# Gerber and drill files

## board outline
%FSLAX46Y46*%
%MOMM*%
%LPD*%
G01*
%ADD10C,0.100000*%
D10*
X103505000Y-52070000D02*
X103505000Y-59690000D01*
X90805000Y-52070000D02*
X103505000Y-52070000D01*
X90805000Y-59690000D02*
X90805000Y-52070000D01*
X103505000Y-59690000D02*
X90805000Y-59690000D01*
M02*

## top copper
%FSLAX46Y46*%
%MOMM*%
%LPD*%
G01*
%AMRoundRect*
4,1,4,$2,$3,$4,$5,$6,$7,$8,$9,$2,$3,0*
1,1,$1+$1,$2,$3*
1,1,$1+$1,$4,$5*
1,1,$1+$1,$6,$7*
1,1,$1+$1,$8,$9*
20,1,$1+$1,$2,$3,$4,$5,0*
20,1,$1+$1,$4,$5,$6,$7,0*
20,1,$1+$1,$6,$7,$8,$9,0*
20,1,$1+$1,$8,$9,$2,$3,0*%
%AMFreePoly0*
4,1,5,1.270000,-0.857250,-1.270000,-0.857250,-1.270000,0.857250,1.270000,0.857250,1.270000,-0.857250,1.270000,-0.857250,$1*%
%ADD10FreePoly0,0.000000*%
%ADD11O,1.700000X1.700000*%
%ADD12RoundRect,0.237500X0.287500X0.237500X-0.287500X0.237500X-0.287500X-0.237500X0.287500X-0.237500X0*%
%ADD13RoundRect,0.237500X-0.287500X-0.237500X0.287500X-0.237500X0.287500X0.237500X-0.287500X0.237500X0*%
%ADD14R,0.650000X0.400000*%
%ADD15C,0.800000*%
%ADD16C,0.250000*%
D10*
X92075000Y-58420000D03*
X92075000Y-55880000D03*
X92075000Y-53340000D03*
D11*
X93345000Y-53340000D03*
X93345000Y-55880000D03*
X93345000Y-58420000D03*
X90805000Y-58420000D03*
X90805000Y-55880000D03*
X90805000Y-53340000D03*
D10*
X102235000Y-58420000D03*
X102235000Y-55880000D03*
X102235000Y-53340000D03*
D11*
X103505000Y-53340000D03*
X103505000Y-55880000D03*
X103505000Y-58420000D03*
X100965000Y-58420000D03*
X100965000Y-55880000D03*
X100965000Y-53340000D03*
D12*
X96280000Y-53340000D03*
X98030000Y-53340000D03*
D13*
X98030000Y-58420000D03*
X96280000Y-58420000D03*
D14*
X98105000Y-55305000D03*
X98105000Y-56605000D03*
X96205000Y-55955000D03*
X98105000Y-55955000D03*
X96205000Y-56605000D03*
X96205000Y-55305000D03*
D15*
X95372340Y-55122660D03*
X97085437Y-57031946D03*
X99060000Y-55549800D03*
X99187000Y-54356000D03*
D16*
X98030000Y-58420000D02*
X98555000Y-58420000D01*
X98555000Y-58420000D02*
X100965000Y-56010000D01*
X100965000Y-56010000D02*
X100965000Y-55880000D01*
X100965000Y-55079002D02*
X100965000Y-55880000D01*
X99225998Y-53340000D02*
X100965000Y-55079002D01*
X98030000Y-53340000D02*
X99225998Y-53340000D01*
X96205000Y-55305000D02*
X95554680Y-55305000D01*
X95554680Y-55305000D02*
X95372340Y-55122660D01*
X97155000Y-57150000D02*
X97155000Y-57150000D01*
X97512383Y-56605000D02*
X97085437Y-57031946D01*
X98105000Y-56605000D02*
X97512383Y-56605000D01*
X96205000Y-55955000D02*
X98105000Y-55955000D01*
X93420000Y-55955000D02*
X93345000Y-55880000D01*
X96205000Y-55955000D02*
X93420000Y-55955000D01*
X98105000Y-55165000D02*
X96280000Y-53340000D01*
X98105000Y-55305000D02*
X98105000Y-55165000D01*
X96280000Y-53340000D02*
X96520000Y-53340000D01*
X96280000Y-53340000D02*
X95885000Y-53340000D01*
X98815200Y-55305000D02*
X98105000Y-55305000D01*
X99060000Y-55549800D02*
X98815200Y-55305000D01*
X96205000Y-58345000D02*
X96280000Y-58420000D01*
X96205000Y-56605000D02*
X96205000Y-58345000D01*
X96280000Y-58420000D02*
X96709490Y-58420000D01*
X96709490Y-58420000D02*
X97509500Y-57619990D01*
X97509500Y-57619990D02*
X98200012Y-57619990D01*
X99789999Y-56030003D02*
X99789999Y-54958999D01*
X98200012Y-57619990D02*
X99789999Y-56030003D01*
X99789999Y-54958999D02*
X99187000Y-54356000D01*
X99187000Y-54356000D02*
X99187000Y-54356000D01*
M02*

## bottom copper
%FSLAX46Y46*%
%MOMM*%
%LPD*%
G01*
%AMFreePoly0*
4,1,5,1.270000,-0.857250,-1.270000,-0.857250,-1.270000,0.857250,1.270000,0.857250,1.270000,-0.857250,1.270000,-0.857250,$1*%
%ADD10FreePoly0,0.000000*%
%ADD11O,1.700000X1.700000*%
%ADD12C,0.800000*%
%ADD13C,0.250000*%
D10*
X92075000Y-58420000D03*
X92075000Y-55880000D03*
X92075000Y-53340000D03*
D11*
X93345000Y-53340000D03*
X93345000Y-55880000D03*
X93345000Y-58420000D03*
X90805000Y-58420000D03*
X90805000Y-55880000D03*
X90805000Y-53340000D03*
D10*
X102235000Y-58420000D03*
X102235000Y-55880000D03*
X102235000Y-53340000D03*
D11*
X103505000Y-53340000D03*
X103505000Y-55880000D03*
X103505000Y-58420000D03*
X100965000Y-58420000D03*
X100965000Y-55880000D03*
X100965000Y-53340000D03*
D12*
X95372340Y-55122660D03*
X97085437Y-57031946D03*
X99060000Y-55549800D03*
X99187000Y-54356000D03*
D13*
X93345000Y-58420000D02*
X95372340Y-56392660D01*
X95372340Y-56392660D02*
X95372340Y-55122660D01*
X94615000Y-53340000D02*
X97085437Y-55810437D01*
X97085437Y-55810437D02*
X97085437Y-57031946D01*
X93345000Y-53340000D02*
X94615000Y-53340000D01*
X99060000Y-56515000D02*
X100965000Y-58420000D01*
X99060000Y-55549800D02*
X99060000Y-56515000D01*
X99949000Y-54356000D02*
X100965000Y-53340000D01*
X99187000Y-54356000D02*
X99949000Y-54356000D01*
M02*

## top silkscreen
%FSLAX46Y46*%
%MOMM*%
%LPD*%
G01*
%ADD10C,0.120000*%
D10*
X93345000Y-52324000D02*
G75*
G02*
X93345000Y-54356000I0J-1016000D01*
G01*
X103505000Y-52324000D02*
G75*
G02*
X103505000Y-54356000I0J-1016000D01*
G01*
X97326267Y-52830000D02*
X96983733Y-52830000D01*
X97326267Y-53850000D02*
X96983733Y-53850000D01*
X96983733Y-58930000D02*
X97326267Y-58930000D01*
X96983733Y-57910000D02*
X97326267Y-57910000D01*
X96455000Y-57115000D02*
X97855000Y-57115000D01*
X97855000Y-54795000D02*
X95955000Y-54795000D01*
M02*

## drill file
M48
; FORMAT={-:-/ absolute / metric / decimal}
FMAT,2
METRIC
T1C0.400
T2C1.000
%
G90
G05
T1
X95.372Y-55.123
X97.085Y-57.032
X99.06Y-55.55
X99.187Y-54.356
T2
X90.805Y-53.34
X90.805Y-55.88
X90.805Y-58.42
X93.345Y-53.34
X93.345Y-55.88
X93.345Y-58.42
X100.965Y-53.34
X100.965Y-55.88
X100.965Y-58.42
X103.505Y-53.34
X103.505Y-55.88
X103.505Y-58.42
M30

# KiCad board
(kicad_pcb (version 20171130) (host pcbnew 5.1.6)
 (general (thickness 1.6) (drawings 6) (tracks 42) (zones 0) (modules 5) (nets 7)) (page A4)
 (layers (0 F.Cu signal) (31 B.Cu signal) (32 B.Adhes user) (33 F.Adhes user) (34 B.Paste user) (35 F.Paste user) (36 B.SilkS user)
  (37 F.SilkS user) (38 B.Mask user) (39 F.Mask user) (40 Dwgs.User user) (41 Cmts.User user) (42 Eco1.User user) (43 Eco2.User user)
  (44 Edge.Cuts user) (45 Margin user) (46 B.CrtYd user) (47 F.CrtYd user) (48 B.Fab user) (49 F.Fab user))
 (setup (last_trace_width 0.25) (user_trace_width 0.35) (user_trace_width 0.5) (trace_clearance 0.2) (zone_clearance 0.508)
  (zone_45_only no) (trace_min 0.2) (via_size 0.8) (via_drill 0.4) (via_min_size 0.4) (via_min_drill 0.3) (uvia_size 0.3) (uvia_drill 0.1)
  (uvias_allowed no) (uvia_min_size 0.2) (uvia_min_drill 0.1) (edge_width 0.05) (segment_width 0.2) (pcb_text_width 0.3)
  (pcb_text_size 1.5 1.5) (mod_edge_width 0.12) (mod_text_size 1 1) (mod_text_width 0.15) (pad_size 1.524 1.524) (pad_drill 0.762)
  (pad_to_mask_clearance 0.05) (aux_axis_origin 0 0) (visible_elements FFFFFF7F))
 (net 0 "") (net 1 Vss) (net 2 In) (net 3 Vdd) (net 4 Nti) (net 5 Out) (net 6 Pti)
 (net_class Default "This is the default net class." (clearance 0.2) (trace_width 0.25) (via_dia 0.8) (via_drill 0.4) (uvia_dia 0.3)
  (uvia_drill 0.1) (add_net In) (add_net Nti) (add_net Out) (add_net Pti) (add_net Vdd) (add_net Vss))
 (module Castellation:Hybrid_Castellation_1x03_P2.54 (layer F.Cu) (at 92.075 53.34)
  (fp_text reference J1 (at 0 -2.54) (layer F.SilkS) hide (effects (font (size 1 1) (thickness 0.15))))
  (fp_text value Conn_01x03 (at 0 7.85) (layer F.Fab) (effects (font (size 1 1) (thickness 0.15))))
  (fp_arc (start 1.27 0) (end 1.27 1.016) (angle -180) (layer F.SilkS) (width 0.12))
  (pad 3 connect custom (at 0 5.08) (size 2.54 1.7145) (layers B.Cu B.Mask) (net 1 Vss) (zone_connect 0)
   (options (clearance outline) (anchor rect)) (primitives))
  (pad 2 connect custom (at 0 2.54) (size 2.54 1.7145) (layers B.Cu B.Mask) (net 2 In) (zone_connect 0)
   (options (clearance outline) (anchor rect)) (primitives))
  (pad 1 connect custom (at 0 0) (size 2.54 1.7145) (layers B.Cu B.Mask) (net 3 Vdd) (zone_connect 0)
   (options (clearance outline) (anchor rect)) (primitives))
  (pad 3 connect custom (at 0 5.08) (size 2.54 1.7145) (layers F.Cu F.Mask) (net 1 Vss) (zone_connect 0)
   (options (clearance outline) (anchor rect)) (primitives))
  (pad 2 connect custom (at 0 2.54) (size 2.54 1.7145) (layers F.Cu F.Mask) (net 2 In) (zone_connect 0)
   (options (clearance outline) (anchor rect)) (primitives))
  (pad 1 connect custom (at 0 0) (size 2.54 1.7145) (layers F.Cu F.Mask) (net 3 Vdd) (zone_connect 0)
   (options (clearance outline) (anchor rect)) (primitives))
  (pad 1 thru_hole oval (at 1.27 0) (size 1.7 1.7) (drill 1) (layers *.Cu *.Mask) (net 3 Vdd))
  (pad 2 thru_hole oval (at 1.27 2.54) (size 1.7 1.7) (drill 1) (layers *.Cu *.Mask) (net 2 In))
  (pad 3 thru_hole oval (at 1.27 5.08) (size 1.7 1.7) (drill 1) (layers *.Cu *.Mask) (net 1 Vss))
  (pad 3 thru_hole oval (at -1.27 5.08) (size 1.7 1.7) (drill 1) (layers *.Cu *.Mask) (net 1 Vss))
  (pad 2 thru_hole oval (at -1.27 2.54) (size 1.7 1.7) (drill 1) (layers *.Cu *.Mask) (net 2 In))
  (pad 1 thru_hole oval (at -1.27 0) (size 1.7 1.7) (drill 1) (layers *.Cu *.Mask) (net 3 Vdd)))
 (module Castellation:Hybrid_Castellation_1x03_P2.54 (layer F.Cu) (at 102.235 53.34)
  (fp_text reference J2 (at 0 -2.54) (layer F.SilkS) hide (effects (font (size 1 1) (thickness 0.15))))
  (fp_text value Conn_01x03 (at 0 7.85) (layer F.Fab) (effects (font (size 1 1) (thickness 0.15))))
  (fp_arc (start 1.27 0) (end 1.27 1.016) (angle -180) (layer F.SilkS) (width 0.12))
  (pad 3 connect custom (at 0 5.08) (size 2.54 1.7145) (layers B.Cu B.Mask) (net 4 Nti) (zone_connect 0)
   (options (clearance outline) (anchor rect)) (primitives))
  (pad 2 connect custom (at 0 2.54) (size 2.54 1.7145) (layers B.Cu B.Mask) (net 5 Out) (zone_connect 0)
   (options (clearance outline) (anchor rect)) (primitives))
  (pad 1 connect custom (at 0 0) (size 2.54 1.7145) (layers B.Cu B.Mask) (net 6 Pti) (zone_connect 0)
   (options (clearance outline) (anchor rect)) (primitives))
  (pad 3 connect custom (at 0 5.08) (size 2.54 1.7145) (layers F.Cu F.Mask) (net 4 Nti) (zone_connect 0)
   (options (clearance outline) (anchor rect)) (primitives))
  (pad 2 connect custom (at 0 2.54) (size 2.54 1.7145) (layers F.Cu F.Mask) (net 5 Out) (zone_connect 0)
   (options (clearance outline) (anchor rect)) (primitives))
  (pad 1 connect custom (at 0 0) (size 2.54 1.7145) (layers F.Cu F.Mask) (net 6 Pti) (zone_connect 0)
   (options (clearance outline) (anchor rect)) (primitives))
  (pad 1 thru_hole oval (at 1.27 0) (size 1.7 1.7) (drill 1) (layers *.Cu *.Mask) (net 6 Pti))
  (pad 2 thru_hole oval (at 1.27 2.54) (size 1.7 1.7) (drill 1) (layers *.Cu *.Mask) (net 5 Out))
  (pad 3 thru_hole oval (at 1.27 5.08) (size 1.7 1.7) (drill 1) (layers *.Cu *.Mask) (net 4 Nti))
  (pad 3 thru_hole oval (at -1.27 5.08) (size 1.7 1.7) (drill 1) (layers *.Cu *.Mask) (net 4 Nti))
  (pad 2 thru_hole oval (at -1.27 2.54) (size 1.7 1.7) (drill 1) (layers *.Cu *.Mask) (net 5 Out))
  (pad 1 thru_hole oval (at -1.27 0) (size 1.7 1.7) (drill 1) (layers *.Cu *.Mask) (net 6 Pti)))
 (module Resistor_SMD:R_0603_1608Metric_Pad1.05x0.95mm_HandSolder (layer F.Cu) (at 97.155 53.34 180)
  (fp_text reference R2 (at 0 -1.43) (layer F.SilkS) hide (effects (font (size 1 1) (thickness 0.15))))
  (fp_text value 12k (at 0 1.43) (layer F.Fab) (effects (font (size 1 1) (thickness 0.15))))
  (fp_line (start -0.171267 0.51) (end 0.171267 0.51) (layer F.SilkS) (width 0.12))
  (fp_line (start -0.171267 -0.51) (end 0.171267 -0.51) (layer F.SilkS) (width 0.12))
  (pad 2 smd roundrect (at 0.875 0 180) (size 1.05 0.95) (layers F.Cu F.Paste F.Mask) (roundrect_rratio 0.25) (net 4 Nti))
  (pad 1 smd roundrect (at -0.875 0 180) (size 1.05 0.95) (layers F.Cu F.Paste F.Mask) (roundrect_rratio 0.25) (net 5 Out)))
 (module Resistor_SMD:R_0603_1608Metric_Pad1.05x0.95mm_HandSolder (layer F.Cu) (at 97.155 58.42)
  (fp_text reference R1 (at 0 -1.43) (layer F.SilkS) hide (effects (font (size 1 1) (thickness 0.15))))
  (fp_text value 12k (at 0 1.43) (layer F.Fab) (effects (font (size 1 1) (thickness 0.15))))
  (fp_line (start -0.171267 0.51) (end 0.171267 0.51) (layer F.SilkS) (width 0.12))
  (fp_line (start -0.171267 -0.51) (end 0.171267 -0.51) (layer F.SilkS) (width 0.12))
  (pad 2 smd roundrect (at 0.875 0) (size 1.05 0.95) (layers F.Cu F.Paste F.Mask) (roundrect_rratio 0.25) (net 5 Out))
  (pad 1 smd roundrect (at -0.875 0) (size 1.05 0.95) (layers F.Cu F.Paste F.Mask) (roundrect_rratio 0.25) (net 6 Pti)))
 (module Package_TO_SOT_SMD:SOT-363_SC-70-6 (layer F.Cu) (at 97.155 55.955)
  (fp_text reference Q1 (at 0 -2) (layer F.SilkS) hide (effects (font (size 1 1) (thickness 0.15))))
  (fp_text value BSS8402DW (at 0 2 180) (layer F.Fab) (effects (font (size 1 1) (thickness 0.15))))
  (fp_line (start -0.7 1.16) (end 0.7 1.16) (layer F.SilkS) (width 0.12))
  (fp_line (start 0.7 -1.16) (end -1.2 -1.16) (layer F.SilkS) (width 0.12))
  (pad 6 smd rect (at 0.95 -0.65) (size 0.65 0.4) (layers F.Cu F.Paste F.Mask) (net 4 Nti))
  (pad 4 smd rect (at 0.95 0.65) (size 0.65 0.4) (layers F.Cu F.Paste F.Mask) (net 3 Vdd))
  (pad 2 smd rect (at -0.95 0) (size 0.65 0.4) (layers F.Cu F.Paste F.Mask) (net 2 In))
  (pad 5 smd rect (at 0.95 0) (size 0.65 0.4) (layers F.Cu F.Paste F.Mask) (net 2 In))
  (pad 3 smd rect (at -0.95 0.65) (size 0.65 0.4) (layers F.Cu F.Paste F.Mask) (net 6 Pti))
  (pad 1 smd rect (at -0.95 -0.65) (size 0.65 0.4) (layers F.Cu F.Paste F.Mask) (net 1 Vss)))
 (gr_line (start 103.505 52.07) (end 103.505 59.69) (layer Edge.Cuts) (width 0.1))
 (gr_line (start 90.805 52.07) (end 103.505 52.07) (layer Edge.Cuts) (width 0.1))
 (gr_line (start 90.805 59.69) (end 90.805 52.07) (layer Edge.Cuts) (width 0.1))
 (gr_line (start 103.505 59.69) (end 90.805 59.69) (layer Edge.Cuts) (width 0.1))
 (segment (start 98.03 58.42) (end 98.555 58.42) (width 0.25) (layer F.Cu) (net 5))
 (segment (start 98.555 58.42) (end 100.965 56.01) (width 0.25) (layer F.Cu) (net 5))
 (segment (start 100.965 56.01) (end 100.965 55.88) (width 0.25) (layer F.Cu) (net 5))
 (segment (start 100.965 55.079002) (end 100.965 55.88) (width 0.25) (layer F.Cu) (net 5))
 (segment (start 99.225998 53.34) (end 100.965 55.079002) (width 0.25) (layer F.Cu) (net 5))
 (segment (start 98.03 53.34) (end 99.225998 53.34) (width 0.25) (layer F.Cu) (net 5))
 (segment (start 96.205 55.305) (end 95.55468 55.305) (width 0.25) (layer F.Cu) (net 1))
 (segment (start 93.345 58.42) (end 95.37234 56.39266) (width 0.25) (layer B.Cu) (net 1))
 (segment (start 95.55468 55.305) (end 95.37234 55.12266) (width 0.25) (layer F.Cu) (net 1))
 (segment (start 95.37234 56.39266) (end 95.37234 55.12266) (width 0.25) (layer B.Cu) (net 1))
 (via (at 95.37234 55.12266) (size 0.8) (drill 0.4) (layers F.Cu B.Cu) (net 1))
 (segment (start 97.155 57.15) (end 97.155 57.15) (width 0.25) (layer F.Cu) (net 3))
 (segment (start 94.615 53.34) (end 97.085437 55.810437) (width 0.25) (layer B.Cu) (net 3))
 (segment (start 97.512383 56.605) (end 97.085437 57.031946) (width 0.25) (layer F.Cu) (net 3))
 (via (at 97.085437 57.031946) (size 0.8) (drill 0.4) (layers F.Cu B.Cu) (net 3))
 (segment (start 98.105 56.605) (end 97.512383 56.605) (width 0.25) (layer F.Cu) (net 3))
 (segment (start 97.085437 55.810437) (end 97.085437 57.031946) (width 0.25) (layer B.Cu) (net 3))
 (segment (start 93.345 53.34) (end 94.615 53.34) (width 0.25) (layer B.Cu) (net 3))
 (segment (start 96.205 55.955) (end 98.105 55.955) (width 0.25) (layer F.Cu) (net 2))
 (segment (start 93.42 55.955) (end 93.345 55.88) (width 0.25) (layer F.Cu) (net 2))
 (segment (start 96.205 55.955) (end 93.42 55.955) (width 0.25) (layer F.Cu) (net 2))
 (via (at 99.06 55.5498) (size 0.8) (drill 0.4) (layers F.Cu B.Cu) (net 4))
 (segment (start 98.105 55.165) (end 96.28 53.34) (width 0.25) (layer F.Cu) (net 4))
 (segment (start 98.105 55.305) (end 98.105 55.165) (width 0.25) (layer F.Cu) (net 4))
 (segment (start 96.28 53.34) (end 96.52 53.34) (width 0.25) (layer F.Cu) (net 4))
 (segment (start 96.28 53.34) (end 95.885 53.34) (width 0.25) (layer F.Cu) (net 4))
 (segment (start 98.8152 55.305) (end 98.105 55.305) (width 0.25) (layer F.Cu) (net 4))
 (segment (start 99.06 55.5498) (end 98.8152 55.305) (width 0.25) (layer F.Cu) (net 4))
 (segment (start 99.06 56.515) (end 100.965 58.42) (width 0.25) (layer B.Cu) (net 4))
 (segment (start 99.06 55.5498) (end 99.06 56.515) (width 0.25) (layer B.Cu) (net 4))
 (segment (start 96.205 58.345) (end 96.28 58.42) (width 0.25) (layer F.Cu) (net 6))
 (segment (start 96.205 56.605) (end 96.205 58.345) (width 0.25) (layer F.Cu) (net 6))
 (segment (start 96.28 58.42) (end 96.70949 58.42) (width 0.25) (layer F.Cu) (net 6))
 (segment (start 96.70949 58.42) (end 97.5095 57.61999) (width 0.25) (layer F.Cu) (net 6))
 (segment (start 97.5095 57.61999) (end 98.200012 57.61999) (width 0.25) (layer F.Cu) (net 6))
 (segment (start 99.789999 56.030003) (end 99.789999 54.958999) (width 0.25) (layer F.Cu) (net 6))
 (segment (start 98.200012 57.61999) (end 99.789999 56.030003) (width 0.25) (layer F.Cu) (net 6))
 (segment (start 99.789999 54.958999) (end 99.187 54.356) (width 0.25) (layer F.Cu) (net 6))
 (segment (start 99.187 54.356) (end 99.187 54.356) (width 0.25) (layer F.Cu) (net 6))
 (via (at 99.187 54.356) (size 0.8) (drill 0.4) (layers F.Cu B.Cu) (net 6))
 (segment (start 99.949 54.356) (end 100.965 53.34) (width 0.25) (layer B.Cu) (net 6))
 (segment (start 99.187 54.356) (end 99.949 54.356) (width 0.25) (layer B.Cu) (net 6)))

